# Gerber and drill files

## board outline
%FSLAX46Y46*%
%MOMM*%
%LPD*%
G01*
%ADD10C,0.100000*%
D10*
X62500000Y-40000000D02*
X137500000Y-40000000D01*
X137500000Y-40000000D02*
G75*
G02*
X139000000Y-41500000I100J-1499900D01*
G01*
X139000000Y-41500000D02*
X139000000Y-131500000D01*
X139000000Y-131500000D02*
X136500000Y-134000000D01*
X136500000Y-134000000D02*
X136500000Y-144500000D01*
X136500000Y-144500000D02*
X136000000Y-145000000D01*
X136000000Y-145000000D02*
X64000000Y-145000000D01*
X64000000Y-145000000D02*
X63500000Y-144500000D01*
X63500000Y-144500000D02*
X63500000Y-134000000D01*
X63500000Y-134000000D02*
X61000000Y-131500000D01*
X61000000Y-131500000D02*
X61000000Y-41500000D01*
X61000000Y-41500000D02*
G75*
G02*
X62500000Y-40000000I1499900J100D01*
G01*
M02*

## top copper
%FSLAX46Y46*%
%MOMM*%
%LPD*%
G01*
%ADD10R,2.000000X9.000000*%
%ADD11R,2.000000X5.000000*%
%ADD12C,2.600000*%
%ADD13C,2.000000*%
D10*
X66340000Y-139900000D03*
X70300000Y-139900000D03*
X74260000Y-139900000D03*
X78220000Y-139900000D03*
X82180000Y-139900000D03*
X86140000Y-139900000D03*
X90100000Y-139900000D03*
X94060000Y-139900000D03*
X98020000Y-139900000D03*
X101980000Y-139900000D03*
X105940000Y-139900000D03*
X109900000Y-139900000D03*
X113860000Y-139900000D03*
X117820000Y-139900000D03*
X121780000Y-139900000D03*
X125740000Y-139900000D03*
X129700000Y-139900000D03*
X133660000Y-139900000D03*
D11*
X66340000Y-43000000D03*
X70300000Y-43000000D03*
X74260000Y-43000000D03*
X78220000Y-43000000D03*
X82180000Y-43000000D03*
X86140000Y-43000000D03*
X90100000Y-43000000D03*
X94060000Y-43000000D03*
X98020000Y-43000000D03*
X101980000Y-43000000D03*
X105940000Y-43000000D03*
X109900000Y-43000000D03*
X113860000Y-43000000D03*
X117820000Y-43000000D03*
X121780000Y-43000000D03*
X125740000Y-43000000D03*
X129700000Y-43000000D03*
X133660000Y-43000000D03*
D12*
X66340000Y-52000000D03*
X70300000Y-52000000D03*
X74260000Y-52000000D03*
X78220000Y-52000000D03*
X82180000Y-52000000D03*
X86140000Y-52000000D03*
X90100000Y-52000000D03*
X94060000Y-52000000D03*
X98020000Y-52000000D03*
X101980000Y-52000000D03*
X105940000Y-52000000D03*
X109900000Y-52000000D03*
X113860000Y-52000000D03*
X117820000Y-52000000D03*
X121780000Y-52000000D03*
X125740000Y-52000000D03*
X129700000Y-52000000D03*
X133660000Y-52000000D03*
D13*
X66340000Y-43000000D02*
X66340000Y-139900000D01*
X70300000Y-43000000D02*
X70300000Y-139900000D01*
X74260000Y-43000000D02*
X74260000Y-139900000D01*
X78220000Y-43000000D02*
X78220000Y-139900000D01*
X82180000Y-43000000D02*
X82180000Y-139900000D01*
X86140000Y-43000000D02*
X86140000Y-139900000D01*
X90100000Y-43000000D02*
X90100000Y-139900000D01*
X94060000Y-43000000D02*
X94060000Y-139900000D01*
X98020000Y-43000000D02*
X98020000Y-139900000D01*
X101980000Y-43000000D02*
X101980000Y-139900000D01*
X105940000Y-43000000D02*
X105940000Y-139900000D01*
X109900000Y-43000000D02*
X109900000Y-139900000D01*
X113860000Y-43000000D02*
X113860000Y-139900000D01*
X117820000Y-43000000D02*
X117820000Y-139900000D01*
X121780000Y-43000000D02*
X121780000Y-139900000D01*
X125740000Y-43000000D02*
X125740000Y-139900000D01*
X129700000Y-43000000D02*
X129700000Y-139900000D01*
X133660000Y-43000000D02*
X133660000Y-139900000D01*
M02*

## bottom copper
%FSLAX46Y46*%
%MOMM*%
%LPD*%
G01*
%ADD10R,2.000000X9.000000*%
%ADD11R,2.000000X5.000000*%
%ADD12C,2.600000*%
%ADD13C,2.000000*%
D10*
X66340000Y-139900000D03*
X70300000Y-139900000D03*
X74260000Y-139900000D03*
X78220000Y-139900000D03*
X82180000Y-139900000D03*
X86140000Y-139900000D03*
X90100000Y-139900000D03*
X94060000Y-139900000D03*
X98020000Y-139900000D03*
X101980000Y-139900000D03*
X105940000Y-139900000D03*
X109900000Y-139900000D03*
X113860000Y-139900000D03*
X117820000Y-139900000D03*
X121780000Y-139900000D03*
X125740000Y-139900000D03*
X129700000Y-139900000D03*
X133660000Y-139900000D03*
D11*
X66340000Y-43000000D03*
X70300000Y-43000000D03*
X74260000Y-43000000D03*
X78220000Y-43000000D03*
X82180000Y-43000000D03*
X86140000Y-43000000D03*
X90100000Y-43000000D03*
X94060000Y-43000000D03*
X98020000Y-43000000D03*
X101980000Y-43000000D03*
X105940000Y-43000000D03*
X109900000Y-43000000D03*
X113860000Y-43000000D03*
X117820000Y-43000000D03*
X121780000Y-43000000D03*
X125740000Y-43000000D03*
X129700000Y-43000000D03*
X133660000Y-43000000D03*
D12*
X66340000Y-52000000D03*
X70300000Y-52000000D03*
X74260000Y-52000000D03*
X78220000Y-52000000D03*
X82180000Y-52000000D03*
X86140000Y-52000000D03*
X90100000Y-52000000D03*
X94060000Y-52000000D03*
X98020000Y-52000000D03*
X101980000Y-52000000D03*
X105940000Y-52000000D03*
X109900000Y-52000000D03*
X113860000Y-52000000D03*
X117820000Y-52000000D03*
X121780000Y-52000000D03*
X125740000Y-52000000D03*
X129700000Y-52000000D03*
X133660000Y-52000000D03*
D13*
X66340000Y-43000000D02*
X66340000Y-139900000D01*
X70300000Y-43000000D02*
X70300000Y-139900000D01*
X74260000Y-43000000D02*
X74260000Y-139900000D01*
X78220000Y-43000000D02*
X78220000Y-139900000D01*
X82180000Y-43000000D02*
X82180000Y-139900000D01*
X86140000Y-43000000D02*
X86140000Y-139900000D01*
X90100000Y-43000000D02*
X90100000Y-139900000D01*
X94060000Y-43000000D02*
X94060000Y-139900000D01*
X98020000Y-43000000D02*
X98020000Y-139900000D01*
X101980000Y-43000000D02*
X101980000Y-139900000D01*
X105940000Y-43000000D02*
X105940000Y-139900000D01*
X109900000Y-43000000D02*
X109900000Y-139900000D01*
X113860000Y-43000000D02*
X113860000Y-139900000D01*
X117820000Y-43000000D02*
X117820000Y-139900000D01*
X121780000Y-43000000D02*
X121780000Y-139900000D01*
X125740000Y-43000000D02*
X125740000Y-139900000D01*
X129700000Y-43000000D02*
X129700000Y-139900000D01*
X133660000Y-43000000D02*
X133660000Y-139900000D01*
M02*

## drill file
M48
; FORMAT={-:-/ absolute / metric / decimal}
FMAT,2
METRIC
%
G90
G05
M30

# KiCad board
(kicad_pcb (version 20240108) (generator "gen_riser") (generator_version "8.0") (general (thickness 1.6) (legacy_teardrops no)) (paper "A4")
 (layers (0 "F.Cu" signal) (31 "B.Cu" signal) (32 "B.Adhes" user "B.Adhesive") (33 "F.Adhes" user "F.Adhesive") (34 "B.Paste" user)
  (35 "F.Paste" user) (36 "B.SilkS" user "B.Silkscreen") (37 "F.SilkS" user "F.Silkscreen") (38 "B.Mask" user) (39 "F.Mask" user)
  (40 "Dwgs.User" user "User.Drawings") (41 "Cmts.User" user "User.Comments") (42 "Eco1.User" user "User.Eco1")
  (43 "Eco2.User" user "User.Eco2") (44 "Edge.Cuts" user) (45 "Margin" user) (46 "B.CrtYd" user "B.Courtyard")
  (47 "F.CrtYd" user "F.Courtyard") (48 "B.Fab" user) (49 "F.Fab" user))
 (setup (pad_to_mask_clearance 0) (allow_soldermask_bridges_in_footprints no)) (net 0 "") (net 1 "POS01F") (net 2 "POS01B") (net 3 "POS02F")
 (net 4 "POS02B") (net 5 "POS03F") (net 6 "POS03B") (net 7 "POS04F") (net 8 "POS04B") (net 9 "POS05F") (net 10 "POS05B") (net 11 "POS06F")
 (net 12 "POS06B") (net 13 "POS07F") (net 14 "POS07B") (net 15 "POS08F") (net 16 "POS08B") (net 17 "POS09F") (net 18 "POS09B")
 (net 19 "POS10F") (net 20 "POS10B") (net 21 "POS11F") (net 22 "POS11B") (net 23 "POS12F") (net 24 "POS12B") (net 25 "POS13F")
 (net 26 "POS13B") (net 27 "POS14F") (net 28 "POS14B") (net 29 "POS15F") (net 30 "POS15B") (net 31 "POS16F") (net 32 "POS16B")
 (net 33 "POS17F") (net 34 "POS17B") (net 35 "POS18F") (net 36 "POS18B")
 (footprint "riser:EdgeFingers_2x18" (layer "F.Cu") (at 100 40)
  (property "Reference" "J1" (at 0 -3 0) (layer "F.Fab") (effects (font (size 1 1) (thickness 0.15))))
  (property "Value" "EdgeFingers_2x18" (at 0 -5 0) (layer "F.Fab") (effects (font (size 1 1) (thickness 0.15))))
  (pad "1" smd rect (at -33.66 99.9) (size 2 9) (layers "F.Cu" "F.Mask") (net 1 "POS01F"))
  (pad "1B" smd rect (at -33.66 99.9) (size 2 9) (layers "B.Cu" "B.Mask") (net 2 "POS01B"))
  (pad "2" smd rect (at -29.7 99.9) (size 2 9) (layers "F.Cu" "F.Mask") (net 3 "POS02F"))
  (pad "2B" smd rect (at -29.7 99.9) (size 2 9) (layers "B.Cu" "B.Mask") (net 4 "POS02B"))
  (pad "3" smd rect (at -25.74 99.9) (size 2 9) (layers "F.Cu" "F.Mask") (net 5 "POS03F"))
  (pad "3B" smd rect (at -25.74 99.9) (size 2 9) (layers "B.Cu" "B.Mask") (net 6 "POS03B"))
  (pad "4" smd rect (at -21.78 99.9) (size 2 9) (layers "F.Cu" "F.Mask") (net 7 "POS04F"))
  (pad "4B" smd rect (at -21.78 99.9) (size 2 9) (layers "B.Cu" "B.Mask") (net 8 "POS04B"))
  (pad "5" smd rect (at -17.82 99.9) (size 2 9) (layers "F.Cu" "F.Mask") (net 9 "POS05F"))
  (pad "5B" smd rect (at -17.82 99.9) (size 2 9) (layers "B.Cu" "B.Mask") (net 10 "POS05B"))
  (pad "6" smd rect (at -13.86 99.9) (size 2 9) (layers "F.Cu" "F.Mask") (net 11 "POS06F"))
  (pad "6B" smd rect (at -13.86 99.9) (size 2 9) (layers "B.Cu" "B.Mask") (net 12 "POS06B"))
  (pad "7" smd rect (at -9.9 99.9) (size 2 9) (layers "F.Cu" "F.Mask") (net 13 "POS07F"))
  (pad "7B" smd rect (at -9.9 99.9) (size 2 9) (layers "B.Cu" "B.Mask") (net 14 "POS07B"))
  (pad "8" smd rect (at -5.94 99.9) (size 2 9) (layers "F.Cu" "F.Mask") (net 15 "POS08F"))
  (pad "8B" smd rect (at -5.94 99.9) (size 2 9) (layers "B.Cu" "B.Mask") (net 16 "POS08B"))
  (pad "9" smd rect (at -1.98 99.9) (size 2 9) (layers "F.Cu" "F.Mask") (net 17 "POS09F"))
  (pad "9B" smd rect (at -1.98 99.9) (size 2 9) (layers "B.Cu" "B.Mask") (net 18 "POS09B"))
  (pad "10" smd rect (at 1.98 99.9) (size 2 9) (layers "F.Cu" "F.Mask") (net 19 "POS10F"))
  (pad "10B" smd rect (at 1.98 99.9) (size 2 9) (layers "B.Cu" "B.Mask") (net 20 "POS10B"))
  (pad "11" smd rect (at 5.94 99.9) (size 2 9) (layers "F.Cu" "F.Mask") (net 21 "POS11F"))
  (pad "11B" smd rect (at 5.94 99.9) (size 2 9) (layers "B.Cu" "B.Mask") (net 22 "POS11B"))
  (pad "12" smd rect (at 9.9 99.9) (size 2 9) (layers "F.Cu" "F.Mask") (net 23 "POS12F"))
  (pad "12B" smd rect (at 9.9 99.9) (size 2 9) (layers "B.Cu" "B.Mask") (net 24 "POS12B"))
  (pad "13" smd rect (at 13.86 99.9) (size 2 9) (layers "F.Cu" "F.Mask") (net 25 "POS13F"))
  (pad "13B" smd rect (at 13.86 99.9) (size 2 9) (layers "B.Cu" "B.Mask") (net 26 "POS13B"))
  (pad "14" smd rect (at 17.82 99.9) (size 2 9) (layers "F.Cu" "F.Mask") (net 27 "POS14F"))
  (pad "14B" smd rect (at 17.82 99.9) (size 2 9) (layers "B.Cu" "B.Mask") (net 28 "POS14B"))
  (pad "15" smd rect (at 21.78 99.9) (size 2 9) (layers "F.Cu" "F.Mask") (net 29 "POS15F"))
  (pad "15B" smd rect (at 21.78 99.9) (size 2 9) (layers "B.Cu" "B.Mask") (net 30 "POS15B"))
  (pad "16" smd rect (at 25.74 99.9) (size 2 9) (layers "F.Cu" "F.Mask") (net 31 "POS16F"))
  (pad "16B" smd rect (at 25.74 99.9) (size 2 9) (layers "B.Cu" "B.Mask") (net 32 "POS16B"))
  (pad "17" smd rect (at 29.7 99.9) (size 2 9) (layers "F.Cu" "F.Mask") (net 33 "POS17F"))
  (pad "17B" smd rect (at 29.7 99.9) (size 2 9) (layers "B.Cu" "B.Mask") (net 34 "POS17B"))
  (pad "18" smd rect (at 33.66 99.9) (size 2 9) (layers "F.Cu" "F.Mask") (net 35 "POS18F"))
  (pad "18B" smd rect (at 33.66 99.9) (size 2 9) (layers "B.Cu" "B.Mask") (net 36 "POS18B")))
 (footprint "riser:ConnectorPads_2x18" (layer "F.Cu") (at 100 40)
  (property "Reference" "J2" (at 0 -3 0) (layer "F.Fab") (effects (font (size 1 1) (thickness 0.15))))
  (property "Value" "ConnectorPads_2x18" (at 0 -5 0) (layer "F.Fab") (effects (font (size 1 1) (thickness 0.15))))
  (pad "1" smd rect (at -33.66 3) (size 2 5) (layers "F.Cu" "F.Mask") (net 1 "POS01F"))
  (pad "1B" smd rect (at -33.66 3) (size 2 5) (layers "B.Cu" "B.Mask") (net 2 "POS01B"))
  (pad "2" smd rect (at -29.7 3) (size 2 5) (layers "F.Cu" "F.Mask") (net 3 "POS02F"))
  (pad "2B" smd rect (at -29.7 3) (size 2 5) (layers "B.Cu" "B.Mask") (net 4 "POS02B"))
  (pad "3" smd rect (at -25.74 3) (size 2 5) (layers "F.Cu" "F.Mask") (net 5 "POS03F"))
  (pad "3B" smd rect (at -25.74 3) (size 2 5) (layers "B.Cu" "B.Mask") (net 6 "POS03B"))
  (pad "4" smd rect (at -21.78 3) (size 2 5) (layers "F.Cu" "F.Mask") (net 7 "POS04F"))
  (pad "4B" smd rect (at -21.78 3) (size 2 5) (layers "B.Cu" "B.Mask") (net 8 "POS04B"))
  (pad "5" smd rect (at -17.82 3) (size 2 5) (layers "F.Cu" "F.Mask") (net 9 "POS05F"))
  (pad "5B" smd rect (at -17.82 3) (size 2 5) (layers "B.Cu" "B.Mask") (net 10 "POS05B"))
  (pad "6" smd rect (at -13.86 3) (size 2 5) (layers "F.Cu" "F.Mask") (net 11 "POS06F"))
  (pad "6B" smd rect (at -13.86 3) (size 2 5) (layers "B.Cu" "B.Mask") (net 12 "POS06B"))
  (pad "7" smd rect (at -9.9 3) (size 2 5) (layers "F.Cu" "F.Mask") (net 13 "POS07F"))
  (pad "7B" smd rect (at -9.9 3) (size 2 5) (layers "B.Cu" "B.Mask") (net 14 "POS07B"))
  (pad "8" smd rect (at -5.94 3) (size 2 5) (layers "F.Cu" "F.Mask") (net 15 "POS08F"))
  (pad "8B" smd rect (at -5.94 3) (size 2 5) (layers "B.Cu" "B.Mask") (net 16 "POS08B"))
  (pad "9" smd rect (at -1.98 3) (size 2 5) (layers "F.Cu" "F.Mask") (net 17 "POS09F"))
  (pad "9B" smd rect (at -1.98 3) (size 2 5) (layers "B.Cu" "B.Mask") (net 18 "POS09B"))
  (pad "10" smd rect (at 1.98 3) (size 2 5) (layers "F.Cu" "F.Mask") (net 19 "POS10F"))
  (pad "10B" smd rect (at 1.98 3) (size 2 5) (layers "B.Cu" "B.Mask") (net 20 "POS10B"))
  (pad "11" smd rect (at 5.94 3) (size 2 5) (layers "F.Cu" "F.Mask") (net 21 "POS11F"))
  (pad "11B" smd rect (at 5.94 3) (size 2 5) (layers "B.Cu" "B.Mask") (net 22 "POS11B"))
  (pad "12" smd rect (at 9.9 3) (size 2 5) (layers "F.Cu" "F.Mask") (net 23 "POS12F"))
  (pad "12B" smd rect (at 9.9 3) (size 2 5) (layers "B.Cu" "B.Mask") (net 24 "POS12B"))
  (pad "13" smd rect (at 13.86 3) (size 2 5) (layers "F.Cu" "F.Mask") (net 25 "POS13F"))
  (pad "13B" smd rect (at 13.86 3) (size 2 5) (layers "B.Cu" "B.Mask") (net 26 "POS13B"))
  (pad "14" smd rect (at 17.82 3) (size 2 5) (layers "F.Cu" "F.Mask") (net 27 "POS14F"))
  (pad "14B" smd rect (at 17.82 3) (size 2 5) (layers "B.Cu" "B.Mask") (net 28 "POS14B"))
  (pad "15" smd rect (at 21.78 3) (size 2 5) (layers "F.Cu" "F.Mask") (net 29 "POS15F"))
  (pad "15B" smd rect (at 21.78 3) (size 2 5) (layers "B.Cu" "B.Mask") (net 30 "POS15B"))
  (pad "16" smd rect (at 25.74 3) (size 2 5) (layers "F.Cu" "F.Mask") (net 31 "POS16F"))
  (pad "16B" smd rect (at 25.74 3) (size 2 5) (layers "B.Cu" "B.Mask") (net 32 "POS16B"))
  (pad "17" smd rect (at 29.7 3) (size 2 5) (layers "F.Cu" "F.Mask") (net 33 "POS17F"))
  (pad "17B" smd rect (at 29.7 3) (size 2 5) (layers "B.Cu" "B.Mask") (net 34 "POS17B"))
  (pad "18" smd rect (at 33.66 3) (size 2 5) (layers "F.Cu" "F.Mask") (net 35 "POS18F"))
  (pad "18B" smd rect (at 33.66 3) (size 2 5) (layers "B.Cu" "B.Mask") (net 36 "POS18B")))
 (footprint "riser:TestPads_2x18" (layer "F.Cu") (at 100 40)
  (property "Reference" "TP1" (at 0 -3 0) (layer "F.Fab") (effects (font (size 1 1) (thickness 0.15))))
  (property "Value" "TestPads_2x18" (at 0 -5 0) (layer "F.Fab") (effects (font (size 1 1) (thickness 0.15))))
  (pad "1" smd circle (at -33.66 12) (size 2.6 2.6) (layers "F.Cu" "F.Mask") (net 1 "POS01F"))
  (pad "1B" smd circle (at -33.66 12) (size 2.6 2.6) (layers "B.Cu" "B.Mask") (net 2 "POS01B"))
  (pad "2" smd circle (at -29.7 12) (size 2.6 2.6) (layers "F.Cu" "F.Mask") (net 3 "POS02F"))
  (pad "2B" smd circle (at -29.7 12) (size 2.6 2.6) (layers "B.Cu" "B.Mask") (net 4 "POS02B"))
  (pad "3" smd circle (at -25.74 12) (size 2.6 2.6) (layers "F.Cu" "F.Mask") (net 5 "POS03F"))
  (pad "3B" smd circle (at -25.74 12) (size 2.6 2.6) (layers "B.Cu" "B.Mask") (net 6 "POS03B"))
  (pad "4" smd circle (at -21.78 12) (size 2.6 2.6) (layers "F.Cu" "F.Mask") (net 7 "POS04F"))
  (pad "4B" smd circle (at -21.78 12) (size 2.6 2.6) (layers "B.Cu" "B.Mask") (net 8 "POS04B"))
  (pad "5" smd circle (at -17.82 12) (size 2.6 2.6) (layers "F.Cu" "F.Mask") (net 9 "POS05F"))
  (pad "5B" smd circle (at -17.82 12) (size 2.6 2.6) (layers "B.Cu" "B.Mask") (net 10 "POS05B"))
  (pad "6" smd circle (at -13.86 12) (size 2.6 2.6) (layers "F.Cu" "F.Mask") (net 11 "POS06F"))
  (pad "6B" smd circle (at -13.86 12) (size 2.6 2.6) (layers "B.Cu" "B.Mask") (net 12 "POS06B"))
  (pad "7" smd circle (at -9.9 12) (size 2.6 2.6) (layers "F.Cu" "F.Mask") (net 13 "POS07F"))
  (pad "7B" smd circle (at -9.9 12) (size 2.6 2.6) (layers "B.Cu" "B.Mask") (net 14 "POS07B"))
  (pad "8" smd circle (at -5.94 12) (size 2.6 2.6) (layers "F.Cu" "F.Mask") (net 15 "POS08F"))
  (pad "8B" smd circle (at -5.94 12) (size 2.6 2.6) (layers "B.Cu" "B.Mask") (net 16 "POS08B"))
  (pad "9" smd circle (at -1.98 12) (size 2.6 2.6) (layers "F.Cu" "F.Mask") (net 17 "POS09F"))
  (pad "9B" smd circle (at -1.98 12) (size 2.6 2.6) (layers "B.Cu" "B.Mask") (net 18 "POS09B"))
  (pad "10" smd circle (at 1.98 12) (size 2.6 2.6) (layers "F.Cu" "F.Mask") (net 19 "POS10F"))
  (pad "10B" smd circle (at 1.98 12) (size 2.6 2.6) (layers "B.Cu" "B.Mask") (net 20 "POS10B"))
  (pad "11" smd circle (at 5.94 12) (size 2.6 2.6) (layers "F.Cu" "F.Mask") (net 21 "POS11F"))
  (pad "11B" smd circle (at 5.94 12) (size 2.6 2.6) (layers "B.Cu" "B.Mask") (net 22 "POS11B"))
  (pad "12" smd circle (at 9.9 12) (size 2.6 2.6) (layers "F.Cu" "F.Mask") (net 23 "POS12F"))
  (pad "12B" smd circle (at 9.9 12) (size 2.6 2.6) (layers "B.Cu" "B.Mask") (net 24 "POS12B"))
  (pad "13" smd circle (at 13.86 12) (size 2.6 2.6) (layers "F.Cu" "F.Mask") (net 25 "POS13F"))
  (pad "13B" smd circle (at 13.86 12) (size 2.6 2.6) (layers "B.Cu" "B.Mask") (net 26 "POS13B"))
  (pad "14" smd circle (at 17.82 12) (size 2.6 2.6) (layers "F.Cu" "F.Mask") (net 27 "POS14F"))
  (pad "14B" smd circle (at 17.82 12) (size 2.6 2.6) (layers "B.Cu" "B.Mask") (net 28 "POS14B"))
  (pad "15" smd circle (at 21.78 12) (size 2.6 2.6) (layers "F.Cu" "F.Mask") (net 29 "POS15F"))
  (pad "15B" smd circle (at 21.78 12) (size 2.6 2.6) (layers "B.Cu" "B.Mask") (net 30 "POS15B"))
  (pad "16" smd circle (at 25.74 12) (size 2.6 2.6) (layers "F.Cu" "F.Mask") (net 31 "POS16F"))
  (pad "16B" smd circle (at 25.74 12) (size 2.6 2.6) (layers "B.Cu" "B.Mask") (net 32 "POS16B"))
  (pad "17" smd circle (at 29.7 12) (size 2.6 2.6) (layers "F.Cu" "F.Mask") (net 33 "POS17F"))
  (pad "17B" smd circle (at 29.7 12) (size 2.6 2.6) (layers "B.Cu" "B.Mask") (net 34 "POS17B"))
  (pad "18" smd circle (at 33.66 12) (size 2.6 2.6) (layers "F.Cu" "F.Mask") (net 35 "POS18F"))
  (pad "18B" smd circle (at 33.66 12) (size 2.6 2.6) (layers "B.Cu" "B.Mask") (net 36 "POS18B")))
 (segment (start 66.34 43) (end 66.34 139.9) (width 2) (layer "F.Cu") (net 1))
 (segment (start 66.34 43) (end 66.34 139.9) (width 2) (layer "B.Cu") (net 2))
 (segment (start 70.3 43) (end 70.3 139.9) (width 2) (layer "F.Cu") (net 3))
 (segment (start 70.3 43) (end 70.3 139.9) (width 2) (layer "B.Cu") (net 4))
 (segment (start 74.26 43) (end 74.26 139.9) (width 2) (layer "F.Cu") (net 5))
 (segment (start 74.26 43) (end 74.26 139.9) (width 2) (layer "B.Cu") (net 6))
 (segment (start 78.22 43) (end 78.22 139.9) (width 2) (layer "F.Cu") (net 7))
 (segment (start 78.22 43) (end 78.22 139.9) (width 2) (layer "B.Cu") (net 8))
 (segment (start 82.18 43) (end 82.18 139.9) (width 2) (layer "F.Cu") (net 9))
 (segment (start 82.18 43) (end 82.18 139.9) (width 2) (layer "B.Cu") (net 10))
 (segment (start 86.14 43) (end 86.14 139.9) (width 2) (layer "F.Cu") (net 11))
 (segment (start 86.14 43) (end 86.14 139.9) (width 2) (layer "B.Cu") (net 12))
 (segment (start 90.1 43) (end 90.1 139.9) (width 2) (layer "F.Cu") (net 13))
 (segment (start 90.1 43) (end 90.1 139.9) (width 2) (layer "B.Cu") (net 14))
 (segment (start 94.06 43) (end 94.06 139.9) (width 2) (layer "F.Cu") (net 15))
 (segment (start 94.06 43) (end 94.06 139.9) (width 2) (layer "B.Cu") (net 16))
 (segment (start 98.02 43) (end 98.02 139.9) (width 2) (layer "F.Cu") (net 17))
 (segment (start 98.02 43) (end 98.02 139.9) (width 2) (layer "B.Cu") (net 18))
 (segment (start 101.98 43) (end 101.98 139.9) (width 2) (layer "F.Cu") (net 19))
 (segment (start 101.98 43) (end 101.98 139.9) (width 2) (layer "B.Cu") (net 20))
 (segment (start 105.94 43) (end 105.94 139.9) (width 2) (layer "F.Cu") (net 21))
 (segment (start 105.94 43) (end 105.94 139.9) (width 2) (layer "B.Cu") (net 22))
 (segment (start 109.9 43) (end 109.9 139.9) (width 2) (layer "F.Cu") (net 23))
 (segment (start 109.9 43) (end 109.9 139.9) (width 2) (layer "B.Cu") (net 24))
 (segment (start 113.86 43) (end 113.86 139.9) (width 2) (layer "F.Cu") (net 25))
 (segment (start 113.86 43) (end 113.86 139.9) (width 2) (layer "B.Cu") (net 26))
 (segment (start 117.82 43) (end 117.82 139.9) (width 2) (layer "F.Cu") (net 27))
 (segment (start 117.82 43) (end 117.82 139.9) (width 2) (layer "B.Cu") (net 28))
 (segment (start 121.78 43) (end 121.78 139.9) (width 2) (layer "F.Cu") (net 29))
 (segment (start 121.78 43) (end 121.78 139.9) (width 2) (layer "B.Cu") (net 30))
 (segment (start 125.74 43) (end 125.74 139.9) (width 2) (layer "F.Cu") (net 31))
 (segment (start 125.74 43) (end 125.74 139.9) (width 2) (layer "B.Cu") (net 32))
 (segment (start 129.7 43) (end 129.7 139.9) (width 2) (layer "F.Cu") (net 33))
 (segment (start 129.7 43) (end 129.7 139.9) (width 2) (layer "B.Cu") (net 34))
 (segment (start 133.66 43) (end 133.66 139.9) (width 2) (layer "F.Cu") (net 35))
 (segment (start 133.66 43) (end 133.66 139.9) (width 2) (layer "B.Cu") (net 36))
 (gr_line (start 62.5 40) (end 137.5 40) (stroke (width 0.1) (type default)) (layer "Edge.Cuts"))
 (gr_arc (start 137.5 40) (mid 138.5607 40.4393) (end 139 41.5) (stroke (width 0.1) (type default)) (layer "Edge.Cuts"))
 (gr_line (start 139 41.5) (end 139 131.5) (stroke (width 0.1) (type default)) (layer "Edge.Cuts"))
 (gr_line (start 139 131.5) (end 136.5 134) (stroke (width 0.1) (type default)) (layer "Edge.Cuts"))
 (gr_line (start 136.5 134) (end 136.5 144.5) (stroke (width 0.1) (type default)) (layer "Edge.Cuts"))
 (gr_line (start 136.5 144.5) (end 136 145) (stroke (width 0.1) (type default)) (layer "Edge.Cuts"))
 (gr_line (start 136 145) (end 64 145) (stroke (width 0.1) (type default)) (layer "Edge.Cuts"))
 (gr_line (start 64 145) (end 63.5 144.5) (stroke (width 0.1) (type default)) (layer "Edge.Cuts"))
 (gr_line (start 63.5 144.5) (end 63.5 134) (stroke (width 0.1) (type default)) (layer "Edge.Cuts"))
 (gr_line (start 63.5 134) (end 61 131.5) (stroke (width 0.1) (type default)) (layer "Edge.Cuts"))
 (gr_line (start 61 131.5) (end 61 41.5) (stroke (width 0.1) (type default)) (layer "Edge.Cuts"))
 (gr_arc (start 61 41.5) (mid 61.4393 40.4393) (end 62.5 40) (stroke (width 0.1) (type default)) (layer "Edge.Cuts")))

